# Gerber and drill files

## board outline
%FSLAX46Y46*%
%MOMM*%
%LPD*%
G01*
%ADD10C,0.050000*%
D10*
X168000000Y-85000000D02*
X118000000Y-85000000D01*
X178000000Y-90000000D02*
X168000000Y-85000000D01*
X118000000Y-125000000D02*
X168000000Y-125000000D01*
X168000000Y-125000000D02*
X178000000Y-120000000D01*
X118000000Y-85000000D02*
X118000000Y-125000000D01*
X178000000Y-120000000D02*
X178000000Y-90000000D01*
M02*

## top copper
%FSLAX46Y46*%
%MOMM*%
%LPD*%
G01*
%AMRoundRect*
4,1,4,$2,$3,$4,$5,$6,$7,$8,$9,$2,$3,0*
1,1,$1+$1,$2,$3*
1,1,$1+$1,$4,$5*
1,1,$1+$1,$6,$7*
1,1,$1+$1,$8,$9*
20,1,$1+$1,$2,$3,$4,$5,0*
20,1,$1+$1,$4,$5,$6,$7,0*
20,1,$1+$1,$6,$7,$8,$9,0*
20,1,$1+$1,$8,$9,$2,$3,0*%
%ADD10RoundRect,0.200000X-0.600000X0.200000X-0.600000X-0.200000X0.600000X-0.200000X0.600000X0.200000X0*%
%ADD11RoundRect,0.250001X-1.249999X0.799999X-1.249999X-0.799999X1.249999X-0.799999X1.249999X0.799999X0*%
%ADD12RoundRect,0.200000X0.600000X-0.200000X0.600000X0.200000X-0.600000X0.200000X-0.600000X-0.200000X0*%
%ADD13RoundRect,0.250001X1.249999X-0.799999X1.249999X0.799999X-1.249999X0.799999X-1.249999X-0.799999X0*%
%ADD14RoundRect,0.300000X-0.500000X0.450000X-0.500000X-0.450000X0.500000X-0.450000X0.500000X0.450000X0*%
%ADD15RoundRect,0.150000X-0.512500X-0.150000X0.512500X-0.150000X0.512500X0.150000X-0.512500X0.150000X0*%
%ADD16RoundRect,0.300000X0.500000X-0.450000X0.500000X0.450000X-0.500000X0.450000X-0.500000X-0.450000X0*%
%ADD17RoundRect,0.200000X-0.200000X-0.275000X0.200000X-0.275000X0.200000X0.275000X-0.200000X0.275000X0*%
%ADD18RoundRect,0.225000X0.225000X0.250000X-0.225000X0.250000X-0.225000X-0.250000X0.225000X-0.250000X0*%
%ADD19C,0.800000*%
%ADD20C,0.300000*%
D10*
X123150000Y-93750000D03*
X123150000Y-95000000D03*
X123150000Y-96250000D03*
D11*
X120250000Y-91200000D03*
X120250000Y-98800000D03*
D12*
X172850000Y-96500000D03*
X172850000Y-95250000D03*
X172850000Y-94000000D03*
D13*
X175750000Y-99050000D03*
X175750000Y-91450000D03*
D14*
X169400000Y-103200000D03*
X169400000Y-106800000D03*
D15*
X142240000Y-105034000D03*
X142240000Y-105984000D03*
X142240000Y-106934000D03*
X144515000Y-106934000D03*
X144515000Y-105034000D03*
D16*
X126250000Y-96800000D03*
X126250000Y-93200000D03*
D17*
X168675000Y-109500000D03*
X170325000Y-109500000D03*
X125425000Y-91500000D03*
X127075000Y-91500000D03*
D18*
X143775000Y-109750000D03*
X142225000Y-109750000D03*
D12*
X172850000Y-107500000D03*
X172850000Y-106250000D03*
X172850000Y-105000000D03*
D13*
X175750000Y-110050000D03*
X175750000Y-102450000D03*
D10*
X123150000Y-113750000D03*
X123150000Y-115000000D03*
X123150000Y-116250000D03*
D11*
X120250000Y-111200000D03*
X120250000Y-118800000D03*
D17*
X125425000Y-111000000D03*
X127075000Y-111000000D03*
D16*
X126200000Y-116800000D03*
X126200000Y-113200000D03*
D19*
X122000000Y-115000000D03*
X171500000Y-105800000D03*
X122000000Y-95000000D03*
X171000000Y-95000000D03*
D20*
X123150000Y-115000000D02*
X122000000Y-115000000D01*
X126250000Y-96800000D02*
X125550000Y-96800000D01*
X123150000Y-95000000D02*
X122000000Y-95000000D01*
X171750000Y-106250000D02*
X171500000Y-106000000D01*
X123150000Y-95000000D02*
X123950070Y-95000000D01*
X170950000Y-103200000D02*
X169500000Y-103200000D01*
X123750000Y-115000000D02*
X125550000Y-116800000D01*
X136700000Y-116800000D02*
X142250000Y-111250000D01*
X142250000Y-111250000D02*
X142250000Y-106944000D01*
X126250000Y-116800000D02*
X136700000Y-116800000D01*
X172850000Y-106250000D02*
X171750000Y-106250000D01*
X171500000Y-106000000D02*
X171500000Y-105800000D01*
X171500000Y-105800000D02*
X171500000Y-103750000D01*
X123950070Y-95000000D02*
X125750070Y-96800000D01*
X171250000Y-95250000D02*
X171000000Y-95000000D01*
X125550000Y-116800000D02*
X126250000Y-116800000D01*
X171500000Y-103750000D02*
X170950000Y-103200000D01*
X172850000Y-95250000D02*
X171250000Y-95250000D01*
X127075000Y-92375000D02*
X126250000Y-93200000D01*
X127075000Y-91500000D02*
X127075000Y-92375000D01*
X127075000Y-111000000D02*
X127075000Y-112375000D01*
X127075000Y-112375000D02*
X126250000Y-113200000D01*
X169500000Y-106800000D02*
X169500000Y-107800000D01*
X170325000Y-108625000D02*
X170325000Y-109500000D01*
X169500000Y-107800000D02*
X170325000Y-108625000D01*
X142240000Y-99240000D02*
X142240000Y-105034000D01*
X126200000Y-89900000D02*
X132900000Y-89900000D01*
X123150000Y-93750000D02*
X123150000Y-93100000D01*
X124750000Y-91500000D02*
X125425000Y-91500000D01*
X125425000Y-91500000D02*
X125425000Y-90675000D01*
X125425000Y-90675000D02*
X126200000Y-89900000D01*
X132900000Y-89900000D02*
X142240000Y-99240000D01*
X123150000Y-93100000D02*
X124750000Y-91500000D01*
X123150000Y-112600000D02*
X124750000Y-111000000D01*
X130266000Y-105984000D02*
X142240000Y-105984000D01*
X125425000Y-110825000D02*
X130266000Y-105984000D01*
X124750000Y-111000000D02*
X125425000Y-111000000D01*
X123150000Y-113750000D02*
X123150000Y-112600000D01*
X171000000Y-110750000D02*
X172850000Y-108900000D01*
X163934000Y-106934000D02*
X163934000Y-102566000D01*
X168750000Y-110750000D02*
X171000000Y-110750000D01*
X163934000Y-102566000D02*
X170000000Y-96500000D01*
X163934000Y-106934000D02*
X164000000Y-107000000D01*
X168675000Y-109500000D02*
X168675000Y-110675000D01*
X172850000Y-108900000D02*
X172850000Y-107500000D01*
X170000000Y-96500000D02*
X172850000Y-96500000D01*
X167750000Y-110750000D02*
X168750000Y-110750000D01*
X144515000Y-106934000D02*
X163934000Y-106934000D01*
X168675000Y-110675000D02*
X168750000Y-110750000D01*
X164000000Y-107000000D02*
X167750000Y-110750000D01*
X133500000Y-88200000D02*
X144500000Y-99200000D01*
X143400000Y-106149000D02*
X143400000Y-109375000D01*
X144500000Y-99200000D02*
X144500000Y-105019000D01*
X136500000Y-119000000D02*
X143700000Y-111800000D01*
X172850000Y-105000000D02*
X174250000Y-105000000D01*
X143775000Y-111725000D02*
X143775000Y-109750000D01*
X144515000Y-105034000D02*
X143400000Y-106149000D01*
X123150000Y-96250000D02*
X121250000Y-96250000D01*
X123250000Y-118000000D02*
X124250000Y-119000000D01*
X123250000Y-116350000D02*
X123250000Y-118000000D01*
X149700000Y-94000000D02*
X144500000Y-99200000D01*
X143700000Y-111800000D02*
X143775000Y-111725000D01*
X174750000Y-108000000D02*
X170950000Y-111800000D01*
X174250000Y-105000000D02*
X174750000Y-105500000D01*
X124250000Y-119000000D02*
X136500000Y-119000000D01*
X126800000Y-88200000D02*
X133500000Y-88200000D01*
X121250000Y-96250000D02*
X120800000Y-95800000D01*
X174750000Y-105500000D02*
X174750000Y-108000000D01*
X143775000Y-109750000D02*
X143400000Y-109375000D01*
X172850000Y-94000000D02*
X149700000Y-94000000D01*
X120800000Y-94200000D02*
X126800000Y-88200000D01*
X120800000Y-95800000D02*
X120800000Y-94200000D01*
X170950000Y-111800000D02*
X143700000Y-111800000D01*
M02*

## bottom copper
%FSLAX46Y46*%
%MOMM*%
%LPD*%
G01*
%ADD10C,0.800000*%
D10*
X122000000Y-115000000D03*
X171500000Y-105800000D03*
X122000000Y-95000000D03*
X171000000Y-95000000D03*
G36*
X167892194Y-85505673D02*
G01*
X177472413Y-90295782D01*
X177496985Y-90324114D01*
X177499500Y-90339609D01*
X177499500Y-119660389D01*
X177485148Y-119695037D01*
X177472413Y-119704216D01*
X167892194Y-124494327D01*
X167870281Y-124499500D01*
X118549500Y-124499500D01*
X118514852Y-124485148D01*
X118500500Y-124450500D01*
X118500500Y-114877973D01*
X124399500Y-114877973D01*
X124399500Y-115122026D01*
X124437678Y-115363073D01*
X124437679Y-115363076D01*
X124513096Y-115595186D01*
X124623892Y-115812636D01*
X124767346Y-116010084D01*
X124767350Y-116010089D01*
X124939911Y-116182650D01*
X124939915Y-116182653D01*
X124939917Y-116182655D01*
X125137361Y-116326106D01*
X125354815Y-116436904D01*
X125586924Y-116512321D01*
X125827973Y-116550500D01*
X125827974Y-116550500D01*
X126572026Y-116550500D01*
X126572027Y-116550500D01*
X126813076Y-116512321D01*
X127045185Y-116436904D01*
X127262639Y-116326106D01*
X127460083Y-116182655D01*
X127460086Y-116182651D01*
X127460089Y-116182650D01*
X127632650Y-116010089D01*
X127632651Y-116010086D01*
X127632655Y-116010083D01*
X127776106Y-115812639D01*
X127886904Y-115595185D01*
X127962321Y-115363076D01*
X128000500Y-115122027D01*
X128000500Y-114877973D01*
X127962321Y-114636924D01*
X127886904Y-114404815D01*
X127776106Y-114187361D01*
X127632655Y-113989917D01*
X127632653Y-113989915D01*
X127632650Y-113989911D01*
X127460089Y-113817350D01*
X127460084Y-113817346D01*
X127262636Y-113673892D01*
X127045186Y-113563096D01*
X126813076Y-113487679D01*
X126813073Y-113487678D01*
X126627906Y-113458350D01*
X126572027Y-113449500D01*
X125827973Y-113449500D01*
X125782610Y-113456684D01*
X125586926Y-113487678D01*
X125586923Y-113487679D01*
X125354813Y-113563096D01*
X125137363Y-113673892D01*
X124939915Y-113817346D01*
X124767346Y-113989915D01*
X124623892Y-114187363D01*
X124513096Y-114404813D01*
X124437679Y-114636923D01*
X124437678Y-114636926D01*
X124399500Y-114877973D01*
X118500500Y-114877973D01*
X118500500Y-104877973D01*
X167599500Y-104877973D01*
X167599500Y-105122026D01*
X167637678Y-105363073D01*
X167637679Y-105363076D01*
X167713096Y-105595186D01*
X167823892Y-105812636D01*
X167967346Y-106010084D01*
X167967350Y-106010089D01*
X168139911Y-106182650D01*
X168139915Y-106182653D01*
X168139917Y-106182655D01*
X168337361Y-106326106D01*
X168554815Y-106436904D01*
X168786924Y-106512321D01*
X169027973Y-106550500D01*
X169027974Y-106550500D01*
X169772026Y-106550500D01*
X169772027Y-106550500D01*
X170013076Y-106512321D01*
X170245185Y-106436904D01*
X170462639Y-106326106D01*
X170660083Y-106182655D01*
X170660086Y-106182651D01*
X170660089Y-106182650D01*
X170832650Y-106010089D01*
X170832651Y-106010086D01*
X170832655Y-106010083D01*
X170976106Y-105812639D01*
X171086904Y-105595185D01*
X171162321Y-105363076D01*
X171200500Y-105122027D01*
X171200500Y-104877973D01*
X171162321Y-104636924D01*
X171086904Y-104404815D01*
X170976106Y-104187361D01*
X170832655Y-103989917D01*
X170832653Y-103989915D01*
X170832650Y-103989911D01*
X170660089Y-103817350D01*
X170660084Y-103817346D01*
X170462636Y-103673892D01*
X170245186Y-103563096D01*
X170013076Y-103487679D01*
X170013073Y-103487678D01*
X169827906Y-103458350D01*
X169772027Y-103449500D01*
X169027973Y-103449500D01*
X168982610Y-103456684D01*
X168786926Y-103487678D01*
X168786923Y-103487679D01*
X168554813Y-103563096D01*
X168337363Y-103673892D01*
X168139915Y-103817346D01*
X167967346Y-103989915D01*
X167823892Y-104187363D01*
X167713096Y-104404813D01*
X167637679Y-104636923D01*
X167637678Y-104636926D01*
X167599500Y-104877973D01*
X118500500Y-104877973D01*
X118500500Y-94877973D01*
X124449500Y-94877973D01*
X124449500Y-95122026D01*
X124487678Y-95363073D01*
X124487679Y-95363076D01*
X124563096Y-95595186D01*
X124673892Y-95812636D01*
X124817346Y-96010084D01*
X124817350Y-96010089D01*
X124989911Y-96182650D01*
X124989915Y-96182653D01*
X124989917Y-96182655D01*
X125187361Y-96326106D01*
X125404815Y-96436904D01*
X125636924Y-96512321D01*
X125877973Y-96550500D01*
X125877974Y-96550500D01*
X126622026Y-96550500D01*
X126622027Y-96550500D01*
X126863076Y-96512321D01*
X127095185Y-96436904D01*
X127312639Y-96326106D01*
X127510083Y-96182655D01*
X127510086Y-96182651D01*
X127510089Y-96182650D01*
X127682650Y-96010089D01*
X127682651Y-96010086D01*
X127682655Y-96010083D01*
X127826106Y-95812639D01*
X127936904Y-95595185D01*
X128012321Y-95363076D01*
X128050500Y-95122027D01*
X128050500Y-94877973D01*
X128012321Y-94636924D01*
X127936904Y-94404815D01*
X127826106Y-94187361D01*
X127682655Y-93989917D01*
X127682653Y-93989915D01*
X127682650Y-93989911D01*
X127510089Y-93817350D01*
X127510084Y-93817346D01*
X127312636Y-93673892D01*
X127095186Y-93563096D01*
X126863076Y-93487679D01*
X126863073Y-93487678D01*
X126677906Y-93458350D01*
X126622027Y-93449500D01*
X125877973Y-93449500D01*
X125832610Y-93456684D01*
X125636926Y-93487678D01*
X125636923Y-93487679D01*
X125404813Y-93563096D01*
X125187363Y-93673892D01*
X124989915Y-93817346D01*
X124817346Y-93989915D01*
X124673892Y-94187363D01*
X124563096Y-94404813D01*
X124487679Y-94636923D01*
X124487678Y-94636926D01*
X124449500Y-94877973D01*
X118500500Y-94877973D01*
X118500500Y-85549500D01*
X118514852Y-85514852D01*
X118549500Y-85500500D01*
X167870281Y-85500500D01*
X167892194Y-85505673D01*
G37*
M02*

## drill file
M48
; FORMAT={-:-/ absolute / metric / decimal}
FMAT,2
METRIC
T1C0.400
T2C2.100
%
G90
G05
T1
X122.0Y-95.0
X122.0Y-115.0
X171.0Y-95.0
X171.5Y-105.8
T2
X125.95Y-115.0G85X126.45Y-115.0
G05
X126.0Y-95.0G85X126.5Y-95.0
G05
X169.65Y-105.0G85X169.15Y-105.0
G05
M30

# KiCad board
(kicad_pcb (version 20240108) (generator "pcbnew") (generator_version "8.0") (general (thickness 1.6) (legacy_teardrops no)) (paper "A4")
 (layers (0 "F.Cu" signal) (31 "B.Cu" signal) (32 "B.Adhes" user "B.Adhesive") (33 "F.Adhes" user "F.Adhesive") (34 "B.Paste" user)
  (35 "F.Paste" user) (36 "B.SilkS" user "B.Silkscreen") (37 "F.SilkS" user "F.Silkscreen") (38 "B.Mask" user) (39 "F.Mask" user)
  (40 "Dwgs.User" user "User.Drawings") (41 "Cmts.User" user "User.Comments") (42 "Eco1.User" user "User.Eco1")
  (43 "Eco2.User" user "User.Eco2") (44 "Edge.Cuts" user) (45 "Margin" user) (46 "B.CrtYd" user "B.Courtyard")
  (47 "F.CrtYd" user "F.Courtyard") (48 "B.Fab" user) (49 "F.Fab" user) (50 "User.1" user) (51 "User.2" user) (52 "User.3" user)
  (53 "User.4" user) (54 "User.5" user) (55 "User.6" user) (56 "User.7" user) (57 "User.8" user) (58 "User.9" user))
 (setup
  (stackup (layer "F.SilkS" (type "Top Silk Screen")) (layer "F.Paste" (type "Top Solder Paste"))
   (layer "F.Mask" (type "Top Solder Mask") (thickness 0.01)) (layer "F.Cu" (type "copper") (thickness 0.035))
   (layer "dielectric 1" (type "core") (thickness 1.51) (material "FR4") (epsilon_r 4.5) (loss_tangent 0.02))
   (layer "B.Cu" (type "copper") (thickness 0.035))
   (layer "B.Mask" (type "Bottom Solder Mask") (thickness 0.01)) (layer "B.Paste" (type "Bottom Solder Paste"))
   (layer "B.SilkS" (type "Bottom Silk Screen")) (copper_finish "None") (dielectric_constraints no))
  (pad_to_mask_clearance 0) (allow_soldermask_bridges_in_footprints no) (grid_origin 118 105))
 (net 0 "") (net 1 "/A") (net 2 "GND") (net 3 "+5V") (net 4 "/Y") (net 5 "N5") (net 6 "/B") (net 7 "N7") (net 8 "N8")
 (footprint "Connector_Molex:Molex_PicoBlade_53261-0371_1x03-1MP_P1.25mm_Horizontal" (layer "F.Cu") (at 120.75 95 -90)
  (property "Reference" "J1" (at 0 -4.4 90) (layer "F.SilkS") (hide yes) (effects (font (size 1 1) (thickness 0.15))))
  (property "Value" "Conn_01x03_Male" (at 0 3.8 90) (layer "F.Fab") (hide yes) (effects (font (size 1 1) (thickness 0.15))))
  (pad "1" smd roundrect (at -1.25 -2.4 270) (size 0.8 1.6) (layers "F.Cu" "F.Paste" "F.Mask") (roundrect_rratio 0.25) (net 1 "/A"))
  (pad "2" smd roundrect (at 0 -2.4 270) (size 0.8 1.6) (layers "F.Cu" "F.Paste" "F.Mask") (roundrect_rratio 0.25) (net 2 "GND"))
  (pad "3" smd roundrect (at 1.25 -2.4 270) (size 0.8 1.6) (layers "F.Cu" "F.Paste" "F.Mask") (roundrect_rratio 0.25) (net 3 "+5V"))
  (pad "MP" smd roundrect (at -3.8 0.5 270) (size 2.1 3) (layers "F.Cu" "F.Paste" "F.Mask") (roundrect_rratio 0.1190480952))
  (pad "MP" smd roundrect (at 3.8 0.5 270) (size 2.1 3) (layers "F.Cu" "F.Paste" "F.Mask") (roundrect_rratio 0.1190480952)))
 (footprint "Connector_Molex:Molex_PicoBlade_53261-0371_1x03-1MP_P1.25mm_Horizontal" (layer "F.Cu") (at 175.25 95.25 90)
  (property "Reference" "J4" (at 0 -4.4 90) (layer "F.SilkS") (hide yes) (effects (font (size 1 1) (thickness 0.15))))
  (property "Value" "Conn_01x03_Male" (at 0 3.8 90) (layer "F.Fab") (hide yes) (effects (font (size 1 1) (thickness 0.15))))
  (pad "1" smd roundrect (at -1.25 -2.4 90) (size 0.8 1.6) (layers "F.Cu" "F.Paste" "F.Mask") (roundrect_rratio 0.25) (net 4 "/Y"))
  (pad "2" smd roundrect (at 0 -2.4 90) (size 0.8 1.6) (layers "F.Cu" "F.Paste" "F.Mask") (roundrect_rratio 0.25) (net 2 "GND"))
  (pad "3" smd roundrect (at 1.25 -2.4 90) (size 0.8 1.6) (layers "F.Cu" "F.Paste" "F.Mask") (roundrect_rratio 0.25) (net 3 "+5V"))
  (pad "MP" smd roundrect (at -3.8 0.5 90) (size 2.1 3) (layers "F.Cu" "F.Paste" "F.Mask") (roundrect_rratio 0.1190480952))
  (pad "MP" smd roundrect (at 3.8 0.5 90) (size 2.1 3) (layers "F.Cu" "F.Paste" "F.Mask") (roundrect_rratio 0.1190480952)))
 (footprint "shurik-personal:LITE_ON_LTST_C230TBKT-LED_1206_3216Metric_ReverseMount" (layer "F.Cu") (at 169.4 105 -90)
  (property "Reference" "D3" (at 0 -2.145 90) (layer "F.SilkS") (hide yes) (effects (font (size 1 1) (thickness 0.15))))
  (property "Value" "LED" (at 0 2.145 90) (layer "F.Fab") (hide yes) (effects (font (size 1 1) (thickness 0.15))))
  (pad "" np_thru_hole oval (at 0 0 270) (size 2.1 2.6) (drill oval 2.1 2.6) (layers "F&B.Cu" "*.Mask"))
  (pad "1" smd roundrect (at -1.8 0 270) (size 1.5 1.6) (layers "F.Cu" "F.Paste" "F.Mask") (roundrect_rratio 0.2) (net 2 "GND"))
  (pad "2" smd roundrect (at 1.8 0 270) (size 1.5 1.6) (layers "F.Cu" "F.Paste" "F.Mask") (roundrect_rratio 0.2) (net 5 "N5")))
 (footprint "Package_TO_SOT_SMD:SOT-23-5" (layer "F.Cu") (at 143.3775 105.984)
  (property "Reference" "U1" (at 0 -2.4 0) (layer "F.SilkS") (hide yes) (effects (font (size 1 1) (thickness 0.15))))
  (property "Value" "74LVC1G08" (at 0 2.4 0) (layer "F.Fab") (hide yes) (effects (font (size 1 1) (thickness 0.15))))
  (pad "1" smd roundrect (at -1.1375 -0.95) (size 1.325 0.6) (layers "F.Cu" "F.Paste" "F.Mask") (roundrect_rratio 0.25) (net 1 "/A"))
  (pad "2" smd roundrect (at -1.1375 0) (size 1.325 0.6) (layers "F.Cu" "F.Paste" "F.Mask") (roundrect_rratio 0.25) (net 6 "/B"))
  (pad "3" smd roundrect (at -1.1375 0.95) (size 1.325 0.6) (layers "F.Cu" "F.Paste" "F.Mask") (roundrect_rratio 0.25) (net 2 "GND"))
  (pad "4" smd roundrect (at 1.1375 0.95) (size 1.325 0.6) (layers "F.Cu" "F.Paste" "F.Mask") (roundrect_rratio 0.25) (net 4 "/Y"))
  (pad "5" smd roundrect (at 1.1375 -0.95) (size 1.325 0.6) (layers "F.Cu" "F.Paste" "F.Mask") (roundrect_rratio 0.25) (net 3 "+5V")))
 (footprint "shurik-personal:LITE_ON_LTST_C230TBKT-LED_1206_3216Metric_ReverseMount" (layer "F.Cu") (at 126.25 95 90)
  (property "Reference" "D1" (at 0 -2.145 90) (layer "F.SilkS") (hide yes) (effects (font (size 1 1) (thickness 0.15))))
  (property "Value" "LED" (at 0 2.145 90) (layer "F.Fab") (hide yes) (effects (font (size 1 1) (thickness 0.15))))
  (pad "" np_thru_hole oval (at 0 0 90) (size 2.1 2.6) (drill oval 2.1 2.6) (layers "F&B.Cu" "*.Mask"))
  (pad "1" smd roundrect (at -1.8 0 90) (size 1.5 1.6) (layers "F.Cu" "F.Paste" "F.Mask") (roundrect_rratio 0.2) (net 2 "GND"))
  (pad "2" smd roundrect (at 1.8 0 90) (size 1.5 1.6) (layers "F.Cu" "F.Paste" "F.Mask") (roundrect_rratio 0.2) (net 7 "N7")))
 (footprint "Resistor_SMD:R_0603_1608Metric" (layer "F.Cu") (at 169.5 109.5)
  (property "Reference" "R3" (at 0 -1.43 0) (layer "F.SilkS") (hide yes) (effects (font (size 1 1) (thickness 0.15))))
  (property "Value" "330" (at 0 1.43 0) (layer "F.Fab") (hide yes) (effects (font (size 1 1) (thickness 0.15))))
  (pad "1" smd roundrect (at -0.825 0) (size 0.8 0.95) (layers "F.Cu" "F.Paste" "F.Mask") (roundrect_rratio 0.25) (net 4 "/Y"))
  (pad "2" smd roundrect (at 0.825 0) (size 0.8 0.95) (layers "F.Cu" "F.Paste" "F.Mask") (roundrect_rratio 0.25) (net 5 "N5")))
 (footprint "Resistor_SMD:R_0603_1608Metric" (layer "F.Cu") (at 126.25 91.5)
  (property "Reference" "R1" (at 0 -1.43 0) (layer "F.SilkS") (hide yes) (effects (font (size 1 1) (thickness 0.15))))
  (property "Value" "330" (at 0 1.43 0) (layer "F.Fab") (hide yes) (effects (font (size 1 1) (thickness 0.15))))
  (pad "1" smd roundrect (at -0.825 0) (size 0.8 0.95) (layers "F.Cu" "F.Paste" "F.Mask") (roundrect_rratio 0.25) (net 1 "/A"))
  (pad "2" smd roundrect (at 0.825 0) (size 0.8 0.95) (layers "F.Cu" "F.Paste" "F.Mask") (roundrect_rratio 0.25) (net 7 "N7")))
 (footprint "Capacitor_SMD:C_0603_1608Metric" (layer "F.Cu") (at 143 109.75 180)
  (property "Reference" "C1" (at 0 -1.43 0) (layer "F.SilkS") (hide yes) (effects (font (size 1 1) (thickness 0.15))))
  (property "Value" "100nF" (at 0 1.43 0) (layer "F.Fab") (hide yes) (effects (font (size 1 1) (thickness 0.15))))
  (pad "1" smd roundrect (at -0.775 0 180) (size 0.9 0.95) (layers "F.Cu" "F.Paste" "F.Mask") (roundrect_rratio 0.25) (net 3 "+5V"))
  (pad "2" smd roundrect (at 0.775 0 180) (size 0.9 0.95) (layers "F.Cu" "F.Paste" "F.Mask") (roundrect_rratio 0.25) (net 2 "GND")))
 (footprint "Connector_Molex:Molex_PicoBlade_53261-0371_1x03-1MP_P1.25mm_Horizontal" (layer "F.Cu") (at 175.25 106.25 90)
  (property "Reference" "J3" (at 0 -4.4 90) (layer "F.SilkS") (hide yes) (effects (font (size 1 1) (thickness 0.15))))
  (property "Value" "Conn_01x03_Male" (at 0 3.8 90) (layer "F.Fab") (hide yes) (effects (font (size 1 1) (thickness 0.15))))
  (pad "1" smd roundrect (at -1.25 -2.4 90) (size 0.8 1.6) (layers "F.Cu" "F.Paste" "F.Mask") (roundrect_rratio 0.25) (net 4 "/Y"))
  (pad "2" smd roundrect (at 0 -2.4 90) (size 0.8 1.6) (layers "F.Cu" "F.Paste" "F.Mask") (roundrect_rratio 0.25) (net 2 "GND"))
  (pad "3" smd roundrect (at 1.25 -2.4 90) (size 0.8 1.6) (layers "F.Cu" "F.Paste" "F.Mask") (roundrect_rratio 0.25) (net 3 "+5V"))
  (pad "MP" smd roundrect (at -3.8 0.5 90) (size 2.1 3) (layers "F.Cu" "F.Paste" "F.Mask") (roundrect_rratio 0.1190480952))
  (pad "MP" smd roundrect (at 3.8 0.5 90) (size 2.1 3) (layers "F.Cu" "F.Paste" "F.Mask") (roundrect_rratio 0.1190480952)))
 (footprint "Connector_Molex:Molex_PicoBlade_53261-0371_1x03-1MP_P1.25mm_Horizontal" (layer "F.Cu") (at 120.75 115 -90)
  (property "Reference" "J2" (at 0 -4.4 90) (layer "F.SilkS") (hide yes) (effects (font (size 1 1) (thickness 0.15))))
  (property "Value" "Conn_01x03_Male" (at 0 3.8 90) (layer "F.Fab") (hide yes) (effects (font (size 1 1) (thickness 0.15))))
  (pad "1" smd roundrect (at -1.25 -2.4 270) (size 0.8 1.6) (layers "F.Cu" "F.Paste" "F.Mask") (roundrect_rratio 0.25) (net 6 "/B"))
  (pad "2" smd roundrect (at 0 -2.4 270) (size 0.8 1.6) (layers "F.Cu" "F.Paste" "F.Mask") (roundrect_rratio 0.25) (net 2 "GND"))
  (pad "3" smd roundrect (at 1.25 -2.4 270) (size 0.8 1.6) (layers "F.Cu" "F.Paste" "F.Mask") (roundrect_rratio 0.25) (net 3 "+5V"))
  (pad "MP" smd roundrect (at -3.8 0.5 270) (size 2.1 3) (layers "F.Cu" "F.Paste" "F.Mask") (roundrect_rratio 0.1190480952))
  (pad "MP" smd roundrect (at 3.8 0.5 270) (size 2.1 3) (layers "F.Cu" "F.Paste" "F.Mask") (roundrect_rratio 0.1190480952)))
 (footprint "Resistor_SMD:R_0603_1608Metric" (layer "F.Cu") (at 126.25 111)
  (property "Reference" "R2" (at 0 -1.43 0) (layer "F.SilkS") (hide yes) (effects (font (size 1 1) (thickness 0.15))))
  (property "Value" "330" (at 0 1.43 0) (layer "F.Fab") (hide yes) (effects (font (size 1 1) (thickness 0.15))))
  (pad "1" smd roundrect (at -0.825 0) (size 0.8 0.95) (layers "F.Cu" "F.Paste" "F.Mask") (roundrect_rratio 0.25) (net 6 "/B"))
  (pad "2" smd roundrect (at 0.825 0) (size 0.8 0.95) (layers "F.Cu" "F.Paste" "F.Mask") (roundrect_rratio 0.25) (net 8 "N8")))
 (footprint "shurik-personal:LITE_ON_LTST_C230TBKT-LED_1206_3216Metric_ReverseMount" (layer "F.Cu") (at 126.2 115 90)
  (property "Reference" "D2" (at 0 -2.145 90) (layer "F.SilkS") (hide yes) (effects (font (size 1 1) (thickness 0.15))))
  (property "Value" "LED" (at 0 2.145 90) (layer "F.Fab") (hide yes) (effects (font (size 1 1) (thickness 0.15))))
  (pad "" np_thru_hole oval (at 0 0 90) (size 2.1 2.6) (drill oval 2.1 2.6) (layers "F&B.Cu" "*.Mask"))
  (pad "1" smd roundrect (at -1.8 0 90) (size 1.5 1.6) (layers "F.Cu" "F.Paste" "F.Mask") (roundrect_rratio 0.2) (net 2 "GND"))
  (pad "2" smd roundrect (at 1.8 0 90) (size 1.5 1.6) (layers "F.Cu" "F.Paste" "F.Mask") (roundrect_rratio 0.2) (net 8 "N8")))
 (gr_line (start 168 85) (end 118 85) (stroke (width 0.05) (type solid)) (layer "Edge.Cuts"))
 (gr_line (start 178 90) (end 168 85) (stroke (width 0.05) (type solid)) (layer "Edge.Cuts"))
 (gr_line (start 118 125) (end 168 125) (stroke (width 0.05) (type solid)) (layer "Edge.Cuts"))
 (gr_line (start 168 125) (end 178 120) (stroke (width 0.05) (type solid)) (layer "Edge.Cuts"))
 (gr_line (start 118 85) (end 118 125) (stroke (width 0.05) (type solid)) (layer "Edge.Cuts"))
 (gr_line (start 178 120) (end 178 90) (stroke (width 0.05) (type solid)) (layer "Edge.Cuts"))
 (segment (start 123.15 115) (end 122 115) (width 0.3) (layer "F.Cu") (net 2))
 (segment (start 126.25 96.8) (end 125.55 96.8) (width 0.3) (layer "F.Cu") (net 2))
 (segment (start 123.15 95) (end 122 95) (width 0.3) (layer "F.Cu") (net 2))
 (segment (start 171.75 106.25) (end 171.5 106) (width 0.3) (layer "F.Cu") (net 2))
 (segment (start 123.15 95) (end 123.95007 95) (width 0.3) (layer "F.Cu") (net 2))
 (segment (start 170.95 103.2) (end 169.5 103.2) (width 0.3) (layer "F.Cu") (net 2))
 (segment (start 123.75 115) (end 125.55 116.8) (width 0.3) (layer "F.Cu") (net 2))
 (segment (start 136.7 116.8) (end 142.25 111.25) (width 0.3) (layer "F.Cu") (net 2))
 (segment (start 142.25 111.25) (end 142.25 106.944) (width 0.3) (layer "F.Cu") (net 2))
 (segment (start 126.25 116.8) (end 136.7 116.8) (width 0.3) (layer "F.Cu") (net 2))
 (segment (start 172.85 106.25) (end 171.75 106.25) (width 0.3) (layer "F.Cu") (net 2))
 (segment (start 171.5 106) (end 171.5 105.8) (width 0.3) (layer "F.Cu") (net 2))
 (segment (start 171.5 105.8) (end 171.5 103.75) (width 0.3) (layer "F.Cu") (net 2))
 (segment (start 123.95007 95) (end 125.75007 96.8) (width 0.3) (layer "F.Cu") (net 2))
 (segment (start 171.25 95.25) (end 171 95) (width 0.3) (layer "F.Cu") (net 2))
 (segment (start 125.55 116.8) (end 126.25 116.8) (width 0.3) (layer "F.Cu") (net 2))
 (segment (start 171.5 103.75) (end 170.95 103.2) (width 0.3) (layer "F.Cu") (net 2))
 (segment (start 172.85 95.25) (end 171.25 95.25) (width 0.3) (layer "F.Cu") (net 2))
 (via (at 122 115) (size 0.8) (drill 0.4) (layers "F.Cu" "B.Cu") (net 2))
 (via (at 171.5 105.8) (size 0.8) (drill 0.4) (layers "F.Cu" "B.Cu") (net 2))
 (via (at 122 95) (size 0.8) (drill 0.4) (layers "F.Cu" "B.Cu") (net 2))
 (via (at 171 95) (size 0.8) (drill 0.4) (layers "F.Cu" "B.Cu") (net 2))
 (segment (start 127.075 92.375) (end 126.25 93.2) (width 0.3) (layer "F.Cu") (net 7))
 (segment (start 127.075 91.5) (end 127.075 92.375) (width 0.3) (layer "F.Cu") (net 7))
 (segment (start 127.075 111) (end 127.075 112.375) (width 0.3) (layer "F.Cu") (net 8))
 (segment (start 127.075 112.375) (end 126.25 113.2) (width 0.3) (layer "F.Cu") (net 8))
 (segment (start 169.5 106.8) (end 169.5 107.8) (width 0.3) (layer "F.Cu") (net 5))
 (segment (start 170.325 108.625) (end 170.325 109.5) (width 0.3) (layer "F.Cu") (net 5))
 (segment (start 169.5 107.8) (end 170.325 108.625) (width 0.3) (layer "F.Cu") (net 5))
 (segment (start 142.24 99.24) (end 142.24 105.034) (width 0.3) (layer "F.Cu") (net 1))
 (segment (start 126.2 89.9) (end 132.9 89.9) (width 0.3) (layer "F.Cu") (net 1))
 (segment (start 123.15 93.75) (end 123.15 93.1) (width 0.3) (layer "F.Cu") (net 1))
 (segment (start 124.75 91.5) (end 125.425 91.5) (width 0.3) (layer "F.Cu") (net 1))
 (segment (start 125.425 91.5) (end 125.425 90.675) (width 0.3) (layer "F.Cu") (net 1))
 (segment (start 125.425 90.675) (end 126.2 89.9) (width 0.3) (layer "F.Cu") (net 1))
 (segment (start 132.9 89.9) (end 142.24 99.24) (width 0.3) (layer "F.Cu") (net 1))
 (segment (start 123.15 93.1) (end 124.75 91.5) (width 0.3) (layer "F.Cu") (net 1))
 (segment (start 123.15 112.6) (end 124.75 111) (width 0.3) (layer "F.Cu") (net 6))
 (segment (start 130.266 105.984) (end 142.24 105.984) (width 0.3) (layer "F.Cu") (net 6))
 (segment (start 125.425 110.825) (end 130.266 105.984) (width 0.3) (layer "F.Cu") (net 6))
 (segment (start 124.75 111) (end 125.425 111) (width 0.3) (layer "F.Cu") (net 6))
 (segment (start 123.15 113.75) (end 123.15 112.6) (width 0.3) (layer "F.Cu") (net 6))
 (segment (start 171 110.75) (end 172.85 108.9) (width 0.3) (layer "F.Cu") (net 4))
 (segment (start 163.934 106.934) (end 163.934 102.566) (width 0.3) (layer "F.Cu") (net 4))
 (segment (start 168.75 110.75) (end 171 110.75) (width 0.3) (layer "F.Cu") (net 4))
 (segment (start 163.934 102.566) (end 170 96.5) (width 0.3) (layer "F.Cu") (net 4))
 (segment (start 163.934 106.934) (end 164 107) (width 0.3) (layer "F.Cu") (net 4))
 (segment (start 168.675 109.5) (end 168.675 110.675) (width 0.3) (layer "F.Cu") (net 4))
 (segment (start 172.85 108.9) (end 172.85 107.5) (width 0.3) (layer "F.Cu") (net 4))
 (segment (start 170 96.5) (end 172.85 96.5) (width 0.3) (layer "F.Cu") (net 4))
 (segment (start 167.75 110.75) (end 168.75 110.75) (width 0.3) (layer "F.Cu") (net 4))
 (segment (start 144.515 106.934) (end 163.934 106.934) (width 0.3) (layer "F.Cu") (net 4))
 (segment (start 168.675 110.675) (end 168.75 110.75) (width 0.3) (layer "F.Cu") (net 4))
 (segment (start 164 107) (end 167.75 110.75) (width 0.3) (layer "F.Cu") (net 4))
 (segment (start 133.5 88.2) (end 144.5 99.2) (width 0.3) (layer "F.Cu") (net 3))
 (segment (start 143.4 106.149) (end 143.4 109.375) (width 0.3) (layer "F.Cu") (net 3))
 (segment (start 144.5 99.2) (end 144.5 105.019) (width 0.3) (layer "F.Cu") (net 3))
 (segment (start 136.5 119) (end 143.7 111.8) (width 0.3) (layer "F.Cu") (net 3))
 (segment (start 172.85 105) (end 174.25 105) (width 0.3) (layer "F.Cu") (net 3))
 (segment (start 143.775 111.725) (end 143.775 109.75) (width 0.3) (layer "F.Cu") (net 3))
 (segment (start 144.515 105.034) (end 143.4 106.149) (width 0.3) (layer "F.Cu") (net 3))
 (segment (start 123.15 96.25) (end 121.25 96.25) (width 0.3) (layer "F.Cu") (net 3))
 (segment (start 123.25 118) (end 124.25 119) (width 0.3) (layer "F.Cu") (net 3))
 (segment (start 123.25 116.35) (end 123.25 118) (width 0.3) (layer "F.Cu") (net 3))
 (segment (start 149.7 94) (end 144.5 99.2) (width 0.3) (layer "F.Cu") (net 3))
 (segment (start 143.7 111.8) (end 143.775 111.725) (width 0.3) (layer "F.Cu") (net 3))
 (segment (start 174.75 108) (end 170.95 111.8) (width 0.3) (layer "F.Cu") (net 3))
 (segment (start 174.25 105) (end 174.75 105.5) (width 0.3) (layer "F.Cu") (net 3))
 (segment (start 124.25 119) (end 136.5 119) (width 0.3) (layer "F.Cu") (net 3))
 (segment (start 126.8 88.2) (end 133.5 88.2) (width 0.3) (layer "F.Cu") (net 3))
 (segment (start 121.25 96.25) (end 120.8 95.8) (width 0.3) (layer "F.Cu") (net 3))
 (segment (start 174.75 105.5) (end 174.75 108) (width 0.3) (layer "F.Cu") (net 3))
 (segment (start 143.775 109.75) (end 143.4 109.375) (width 0.3) (layer "F.Cu") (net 3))
 (segment (start 172.85 94) (end 149.7 94) (width 0.3) (layer "F.Cu") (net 3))
 (segment (start 120.8 94.2) (end 126.8 88.2) (width 0.3) (layer "F.Cu") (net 3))
 (segment (start 120.8 95.8) (end 120.8 94.2) (width 0.3) (layer "F.Cu") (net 3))
 (segment (start 170.95 111.8) (end 143.7 111.8) (width 0.3) (layer "F.Cu") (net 3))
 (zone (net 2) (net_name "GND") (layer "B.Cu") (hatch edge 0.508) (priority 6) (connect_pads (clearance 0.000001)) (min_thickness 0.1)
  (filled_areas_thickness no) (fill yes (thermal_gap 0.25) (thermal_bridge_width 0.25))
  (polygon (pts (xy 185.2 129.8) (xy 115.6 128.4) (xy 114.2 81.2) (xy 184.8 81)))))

